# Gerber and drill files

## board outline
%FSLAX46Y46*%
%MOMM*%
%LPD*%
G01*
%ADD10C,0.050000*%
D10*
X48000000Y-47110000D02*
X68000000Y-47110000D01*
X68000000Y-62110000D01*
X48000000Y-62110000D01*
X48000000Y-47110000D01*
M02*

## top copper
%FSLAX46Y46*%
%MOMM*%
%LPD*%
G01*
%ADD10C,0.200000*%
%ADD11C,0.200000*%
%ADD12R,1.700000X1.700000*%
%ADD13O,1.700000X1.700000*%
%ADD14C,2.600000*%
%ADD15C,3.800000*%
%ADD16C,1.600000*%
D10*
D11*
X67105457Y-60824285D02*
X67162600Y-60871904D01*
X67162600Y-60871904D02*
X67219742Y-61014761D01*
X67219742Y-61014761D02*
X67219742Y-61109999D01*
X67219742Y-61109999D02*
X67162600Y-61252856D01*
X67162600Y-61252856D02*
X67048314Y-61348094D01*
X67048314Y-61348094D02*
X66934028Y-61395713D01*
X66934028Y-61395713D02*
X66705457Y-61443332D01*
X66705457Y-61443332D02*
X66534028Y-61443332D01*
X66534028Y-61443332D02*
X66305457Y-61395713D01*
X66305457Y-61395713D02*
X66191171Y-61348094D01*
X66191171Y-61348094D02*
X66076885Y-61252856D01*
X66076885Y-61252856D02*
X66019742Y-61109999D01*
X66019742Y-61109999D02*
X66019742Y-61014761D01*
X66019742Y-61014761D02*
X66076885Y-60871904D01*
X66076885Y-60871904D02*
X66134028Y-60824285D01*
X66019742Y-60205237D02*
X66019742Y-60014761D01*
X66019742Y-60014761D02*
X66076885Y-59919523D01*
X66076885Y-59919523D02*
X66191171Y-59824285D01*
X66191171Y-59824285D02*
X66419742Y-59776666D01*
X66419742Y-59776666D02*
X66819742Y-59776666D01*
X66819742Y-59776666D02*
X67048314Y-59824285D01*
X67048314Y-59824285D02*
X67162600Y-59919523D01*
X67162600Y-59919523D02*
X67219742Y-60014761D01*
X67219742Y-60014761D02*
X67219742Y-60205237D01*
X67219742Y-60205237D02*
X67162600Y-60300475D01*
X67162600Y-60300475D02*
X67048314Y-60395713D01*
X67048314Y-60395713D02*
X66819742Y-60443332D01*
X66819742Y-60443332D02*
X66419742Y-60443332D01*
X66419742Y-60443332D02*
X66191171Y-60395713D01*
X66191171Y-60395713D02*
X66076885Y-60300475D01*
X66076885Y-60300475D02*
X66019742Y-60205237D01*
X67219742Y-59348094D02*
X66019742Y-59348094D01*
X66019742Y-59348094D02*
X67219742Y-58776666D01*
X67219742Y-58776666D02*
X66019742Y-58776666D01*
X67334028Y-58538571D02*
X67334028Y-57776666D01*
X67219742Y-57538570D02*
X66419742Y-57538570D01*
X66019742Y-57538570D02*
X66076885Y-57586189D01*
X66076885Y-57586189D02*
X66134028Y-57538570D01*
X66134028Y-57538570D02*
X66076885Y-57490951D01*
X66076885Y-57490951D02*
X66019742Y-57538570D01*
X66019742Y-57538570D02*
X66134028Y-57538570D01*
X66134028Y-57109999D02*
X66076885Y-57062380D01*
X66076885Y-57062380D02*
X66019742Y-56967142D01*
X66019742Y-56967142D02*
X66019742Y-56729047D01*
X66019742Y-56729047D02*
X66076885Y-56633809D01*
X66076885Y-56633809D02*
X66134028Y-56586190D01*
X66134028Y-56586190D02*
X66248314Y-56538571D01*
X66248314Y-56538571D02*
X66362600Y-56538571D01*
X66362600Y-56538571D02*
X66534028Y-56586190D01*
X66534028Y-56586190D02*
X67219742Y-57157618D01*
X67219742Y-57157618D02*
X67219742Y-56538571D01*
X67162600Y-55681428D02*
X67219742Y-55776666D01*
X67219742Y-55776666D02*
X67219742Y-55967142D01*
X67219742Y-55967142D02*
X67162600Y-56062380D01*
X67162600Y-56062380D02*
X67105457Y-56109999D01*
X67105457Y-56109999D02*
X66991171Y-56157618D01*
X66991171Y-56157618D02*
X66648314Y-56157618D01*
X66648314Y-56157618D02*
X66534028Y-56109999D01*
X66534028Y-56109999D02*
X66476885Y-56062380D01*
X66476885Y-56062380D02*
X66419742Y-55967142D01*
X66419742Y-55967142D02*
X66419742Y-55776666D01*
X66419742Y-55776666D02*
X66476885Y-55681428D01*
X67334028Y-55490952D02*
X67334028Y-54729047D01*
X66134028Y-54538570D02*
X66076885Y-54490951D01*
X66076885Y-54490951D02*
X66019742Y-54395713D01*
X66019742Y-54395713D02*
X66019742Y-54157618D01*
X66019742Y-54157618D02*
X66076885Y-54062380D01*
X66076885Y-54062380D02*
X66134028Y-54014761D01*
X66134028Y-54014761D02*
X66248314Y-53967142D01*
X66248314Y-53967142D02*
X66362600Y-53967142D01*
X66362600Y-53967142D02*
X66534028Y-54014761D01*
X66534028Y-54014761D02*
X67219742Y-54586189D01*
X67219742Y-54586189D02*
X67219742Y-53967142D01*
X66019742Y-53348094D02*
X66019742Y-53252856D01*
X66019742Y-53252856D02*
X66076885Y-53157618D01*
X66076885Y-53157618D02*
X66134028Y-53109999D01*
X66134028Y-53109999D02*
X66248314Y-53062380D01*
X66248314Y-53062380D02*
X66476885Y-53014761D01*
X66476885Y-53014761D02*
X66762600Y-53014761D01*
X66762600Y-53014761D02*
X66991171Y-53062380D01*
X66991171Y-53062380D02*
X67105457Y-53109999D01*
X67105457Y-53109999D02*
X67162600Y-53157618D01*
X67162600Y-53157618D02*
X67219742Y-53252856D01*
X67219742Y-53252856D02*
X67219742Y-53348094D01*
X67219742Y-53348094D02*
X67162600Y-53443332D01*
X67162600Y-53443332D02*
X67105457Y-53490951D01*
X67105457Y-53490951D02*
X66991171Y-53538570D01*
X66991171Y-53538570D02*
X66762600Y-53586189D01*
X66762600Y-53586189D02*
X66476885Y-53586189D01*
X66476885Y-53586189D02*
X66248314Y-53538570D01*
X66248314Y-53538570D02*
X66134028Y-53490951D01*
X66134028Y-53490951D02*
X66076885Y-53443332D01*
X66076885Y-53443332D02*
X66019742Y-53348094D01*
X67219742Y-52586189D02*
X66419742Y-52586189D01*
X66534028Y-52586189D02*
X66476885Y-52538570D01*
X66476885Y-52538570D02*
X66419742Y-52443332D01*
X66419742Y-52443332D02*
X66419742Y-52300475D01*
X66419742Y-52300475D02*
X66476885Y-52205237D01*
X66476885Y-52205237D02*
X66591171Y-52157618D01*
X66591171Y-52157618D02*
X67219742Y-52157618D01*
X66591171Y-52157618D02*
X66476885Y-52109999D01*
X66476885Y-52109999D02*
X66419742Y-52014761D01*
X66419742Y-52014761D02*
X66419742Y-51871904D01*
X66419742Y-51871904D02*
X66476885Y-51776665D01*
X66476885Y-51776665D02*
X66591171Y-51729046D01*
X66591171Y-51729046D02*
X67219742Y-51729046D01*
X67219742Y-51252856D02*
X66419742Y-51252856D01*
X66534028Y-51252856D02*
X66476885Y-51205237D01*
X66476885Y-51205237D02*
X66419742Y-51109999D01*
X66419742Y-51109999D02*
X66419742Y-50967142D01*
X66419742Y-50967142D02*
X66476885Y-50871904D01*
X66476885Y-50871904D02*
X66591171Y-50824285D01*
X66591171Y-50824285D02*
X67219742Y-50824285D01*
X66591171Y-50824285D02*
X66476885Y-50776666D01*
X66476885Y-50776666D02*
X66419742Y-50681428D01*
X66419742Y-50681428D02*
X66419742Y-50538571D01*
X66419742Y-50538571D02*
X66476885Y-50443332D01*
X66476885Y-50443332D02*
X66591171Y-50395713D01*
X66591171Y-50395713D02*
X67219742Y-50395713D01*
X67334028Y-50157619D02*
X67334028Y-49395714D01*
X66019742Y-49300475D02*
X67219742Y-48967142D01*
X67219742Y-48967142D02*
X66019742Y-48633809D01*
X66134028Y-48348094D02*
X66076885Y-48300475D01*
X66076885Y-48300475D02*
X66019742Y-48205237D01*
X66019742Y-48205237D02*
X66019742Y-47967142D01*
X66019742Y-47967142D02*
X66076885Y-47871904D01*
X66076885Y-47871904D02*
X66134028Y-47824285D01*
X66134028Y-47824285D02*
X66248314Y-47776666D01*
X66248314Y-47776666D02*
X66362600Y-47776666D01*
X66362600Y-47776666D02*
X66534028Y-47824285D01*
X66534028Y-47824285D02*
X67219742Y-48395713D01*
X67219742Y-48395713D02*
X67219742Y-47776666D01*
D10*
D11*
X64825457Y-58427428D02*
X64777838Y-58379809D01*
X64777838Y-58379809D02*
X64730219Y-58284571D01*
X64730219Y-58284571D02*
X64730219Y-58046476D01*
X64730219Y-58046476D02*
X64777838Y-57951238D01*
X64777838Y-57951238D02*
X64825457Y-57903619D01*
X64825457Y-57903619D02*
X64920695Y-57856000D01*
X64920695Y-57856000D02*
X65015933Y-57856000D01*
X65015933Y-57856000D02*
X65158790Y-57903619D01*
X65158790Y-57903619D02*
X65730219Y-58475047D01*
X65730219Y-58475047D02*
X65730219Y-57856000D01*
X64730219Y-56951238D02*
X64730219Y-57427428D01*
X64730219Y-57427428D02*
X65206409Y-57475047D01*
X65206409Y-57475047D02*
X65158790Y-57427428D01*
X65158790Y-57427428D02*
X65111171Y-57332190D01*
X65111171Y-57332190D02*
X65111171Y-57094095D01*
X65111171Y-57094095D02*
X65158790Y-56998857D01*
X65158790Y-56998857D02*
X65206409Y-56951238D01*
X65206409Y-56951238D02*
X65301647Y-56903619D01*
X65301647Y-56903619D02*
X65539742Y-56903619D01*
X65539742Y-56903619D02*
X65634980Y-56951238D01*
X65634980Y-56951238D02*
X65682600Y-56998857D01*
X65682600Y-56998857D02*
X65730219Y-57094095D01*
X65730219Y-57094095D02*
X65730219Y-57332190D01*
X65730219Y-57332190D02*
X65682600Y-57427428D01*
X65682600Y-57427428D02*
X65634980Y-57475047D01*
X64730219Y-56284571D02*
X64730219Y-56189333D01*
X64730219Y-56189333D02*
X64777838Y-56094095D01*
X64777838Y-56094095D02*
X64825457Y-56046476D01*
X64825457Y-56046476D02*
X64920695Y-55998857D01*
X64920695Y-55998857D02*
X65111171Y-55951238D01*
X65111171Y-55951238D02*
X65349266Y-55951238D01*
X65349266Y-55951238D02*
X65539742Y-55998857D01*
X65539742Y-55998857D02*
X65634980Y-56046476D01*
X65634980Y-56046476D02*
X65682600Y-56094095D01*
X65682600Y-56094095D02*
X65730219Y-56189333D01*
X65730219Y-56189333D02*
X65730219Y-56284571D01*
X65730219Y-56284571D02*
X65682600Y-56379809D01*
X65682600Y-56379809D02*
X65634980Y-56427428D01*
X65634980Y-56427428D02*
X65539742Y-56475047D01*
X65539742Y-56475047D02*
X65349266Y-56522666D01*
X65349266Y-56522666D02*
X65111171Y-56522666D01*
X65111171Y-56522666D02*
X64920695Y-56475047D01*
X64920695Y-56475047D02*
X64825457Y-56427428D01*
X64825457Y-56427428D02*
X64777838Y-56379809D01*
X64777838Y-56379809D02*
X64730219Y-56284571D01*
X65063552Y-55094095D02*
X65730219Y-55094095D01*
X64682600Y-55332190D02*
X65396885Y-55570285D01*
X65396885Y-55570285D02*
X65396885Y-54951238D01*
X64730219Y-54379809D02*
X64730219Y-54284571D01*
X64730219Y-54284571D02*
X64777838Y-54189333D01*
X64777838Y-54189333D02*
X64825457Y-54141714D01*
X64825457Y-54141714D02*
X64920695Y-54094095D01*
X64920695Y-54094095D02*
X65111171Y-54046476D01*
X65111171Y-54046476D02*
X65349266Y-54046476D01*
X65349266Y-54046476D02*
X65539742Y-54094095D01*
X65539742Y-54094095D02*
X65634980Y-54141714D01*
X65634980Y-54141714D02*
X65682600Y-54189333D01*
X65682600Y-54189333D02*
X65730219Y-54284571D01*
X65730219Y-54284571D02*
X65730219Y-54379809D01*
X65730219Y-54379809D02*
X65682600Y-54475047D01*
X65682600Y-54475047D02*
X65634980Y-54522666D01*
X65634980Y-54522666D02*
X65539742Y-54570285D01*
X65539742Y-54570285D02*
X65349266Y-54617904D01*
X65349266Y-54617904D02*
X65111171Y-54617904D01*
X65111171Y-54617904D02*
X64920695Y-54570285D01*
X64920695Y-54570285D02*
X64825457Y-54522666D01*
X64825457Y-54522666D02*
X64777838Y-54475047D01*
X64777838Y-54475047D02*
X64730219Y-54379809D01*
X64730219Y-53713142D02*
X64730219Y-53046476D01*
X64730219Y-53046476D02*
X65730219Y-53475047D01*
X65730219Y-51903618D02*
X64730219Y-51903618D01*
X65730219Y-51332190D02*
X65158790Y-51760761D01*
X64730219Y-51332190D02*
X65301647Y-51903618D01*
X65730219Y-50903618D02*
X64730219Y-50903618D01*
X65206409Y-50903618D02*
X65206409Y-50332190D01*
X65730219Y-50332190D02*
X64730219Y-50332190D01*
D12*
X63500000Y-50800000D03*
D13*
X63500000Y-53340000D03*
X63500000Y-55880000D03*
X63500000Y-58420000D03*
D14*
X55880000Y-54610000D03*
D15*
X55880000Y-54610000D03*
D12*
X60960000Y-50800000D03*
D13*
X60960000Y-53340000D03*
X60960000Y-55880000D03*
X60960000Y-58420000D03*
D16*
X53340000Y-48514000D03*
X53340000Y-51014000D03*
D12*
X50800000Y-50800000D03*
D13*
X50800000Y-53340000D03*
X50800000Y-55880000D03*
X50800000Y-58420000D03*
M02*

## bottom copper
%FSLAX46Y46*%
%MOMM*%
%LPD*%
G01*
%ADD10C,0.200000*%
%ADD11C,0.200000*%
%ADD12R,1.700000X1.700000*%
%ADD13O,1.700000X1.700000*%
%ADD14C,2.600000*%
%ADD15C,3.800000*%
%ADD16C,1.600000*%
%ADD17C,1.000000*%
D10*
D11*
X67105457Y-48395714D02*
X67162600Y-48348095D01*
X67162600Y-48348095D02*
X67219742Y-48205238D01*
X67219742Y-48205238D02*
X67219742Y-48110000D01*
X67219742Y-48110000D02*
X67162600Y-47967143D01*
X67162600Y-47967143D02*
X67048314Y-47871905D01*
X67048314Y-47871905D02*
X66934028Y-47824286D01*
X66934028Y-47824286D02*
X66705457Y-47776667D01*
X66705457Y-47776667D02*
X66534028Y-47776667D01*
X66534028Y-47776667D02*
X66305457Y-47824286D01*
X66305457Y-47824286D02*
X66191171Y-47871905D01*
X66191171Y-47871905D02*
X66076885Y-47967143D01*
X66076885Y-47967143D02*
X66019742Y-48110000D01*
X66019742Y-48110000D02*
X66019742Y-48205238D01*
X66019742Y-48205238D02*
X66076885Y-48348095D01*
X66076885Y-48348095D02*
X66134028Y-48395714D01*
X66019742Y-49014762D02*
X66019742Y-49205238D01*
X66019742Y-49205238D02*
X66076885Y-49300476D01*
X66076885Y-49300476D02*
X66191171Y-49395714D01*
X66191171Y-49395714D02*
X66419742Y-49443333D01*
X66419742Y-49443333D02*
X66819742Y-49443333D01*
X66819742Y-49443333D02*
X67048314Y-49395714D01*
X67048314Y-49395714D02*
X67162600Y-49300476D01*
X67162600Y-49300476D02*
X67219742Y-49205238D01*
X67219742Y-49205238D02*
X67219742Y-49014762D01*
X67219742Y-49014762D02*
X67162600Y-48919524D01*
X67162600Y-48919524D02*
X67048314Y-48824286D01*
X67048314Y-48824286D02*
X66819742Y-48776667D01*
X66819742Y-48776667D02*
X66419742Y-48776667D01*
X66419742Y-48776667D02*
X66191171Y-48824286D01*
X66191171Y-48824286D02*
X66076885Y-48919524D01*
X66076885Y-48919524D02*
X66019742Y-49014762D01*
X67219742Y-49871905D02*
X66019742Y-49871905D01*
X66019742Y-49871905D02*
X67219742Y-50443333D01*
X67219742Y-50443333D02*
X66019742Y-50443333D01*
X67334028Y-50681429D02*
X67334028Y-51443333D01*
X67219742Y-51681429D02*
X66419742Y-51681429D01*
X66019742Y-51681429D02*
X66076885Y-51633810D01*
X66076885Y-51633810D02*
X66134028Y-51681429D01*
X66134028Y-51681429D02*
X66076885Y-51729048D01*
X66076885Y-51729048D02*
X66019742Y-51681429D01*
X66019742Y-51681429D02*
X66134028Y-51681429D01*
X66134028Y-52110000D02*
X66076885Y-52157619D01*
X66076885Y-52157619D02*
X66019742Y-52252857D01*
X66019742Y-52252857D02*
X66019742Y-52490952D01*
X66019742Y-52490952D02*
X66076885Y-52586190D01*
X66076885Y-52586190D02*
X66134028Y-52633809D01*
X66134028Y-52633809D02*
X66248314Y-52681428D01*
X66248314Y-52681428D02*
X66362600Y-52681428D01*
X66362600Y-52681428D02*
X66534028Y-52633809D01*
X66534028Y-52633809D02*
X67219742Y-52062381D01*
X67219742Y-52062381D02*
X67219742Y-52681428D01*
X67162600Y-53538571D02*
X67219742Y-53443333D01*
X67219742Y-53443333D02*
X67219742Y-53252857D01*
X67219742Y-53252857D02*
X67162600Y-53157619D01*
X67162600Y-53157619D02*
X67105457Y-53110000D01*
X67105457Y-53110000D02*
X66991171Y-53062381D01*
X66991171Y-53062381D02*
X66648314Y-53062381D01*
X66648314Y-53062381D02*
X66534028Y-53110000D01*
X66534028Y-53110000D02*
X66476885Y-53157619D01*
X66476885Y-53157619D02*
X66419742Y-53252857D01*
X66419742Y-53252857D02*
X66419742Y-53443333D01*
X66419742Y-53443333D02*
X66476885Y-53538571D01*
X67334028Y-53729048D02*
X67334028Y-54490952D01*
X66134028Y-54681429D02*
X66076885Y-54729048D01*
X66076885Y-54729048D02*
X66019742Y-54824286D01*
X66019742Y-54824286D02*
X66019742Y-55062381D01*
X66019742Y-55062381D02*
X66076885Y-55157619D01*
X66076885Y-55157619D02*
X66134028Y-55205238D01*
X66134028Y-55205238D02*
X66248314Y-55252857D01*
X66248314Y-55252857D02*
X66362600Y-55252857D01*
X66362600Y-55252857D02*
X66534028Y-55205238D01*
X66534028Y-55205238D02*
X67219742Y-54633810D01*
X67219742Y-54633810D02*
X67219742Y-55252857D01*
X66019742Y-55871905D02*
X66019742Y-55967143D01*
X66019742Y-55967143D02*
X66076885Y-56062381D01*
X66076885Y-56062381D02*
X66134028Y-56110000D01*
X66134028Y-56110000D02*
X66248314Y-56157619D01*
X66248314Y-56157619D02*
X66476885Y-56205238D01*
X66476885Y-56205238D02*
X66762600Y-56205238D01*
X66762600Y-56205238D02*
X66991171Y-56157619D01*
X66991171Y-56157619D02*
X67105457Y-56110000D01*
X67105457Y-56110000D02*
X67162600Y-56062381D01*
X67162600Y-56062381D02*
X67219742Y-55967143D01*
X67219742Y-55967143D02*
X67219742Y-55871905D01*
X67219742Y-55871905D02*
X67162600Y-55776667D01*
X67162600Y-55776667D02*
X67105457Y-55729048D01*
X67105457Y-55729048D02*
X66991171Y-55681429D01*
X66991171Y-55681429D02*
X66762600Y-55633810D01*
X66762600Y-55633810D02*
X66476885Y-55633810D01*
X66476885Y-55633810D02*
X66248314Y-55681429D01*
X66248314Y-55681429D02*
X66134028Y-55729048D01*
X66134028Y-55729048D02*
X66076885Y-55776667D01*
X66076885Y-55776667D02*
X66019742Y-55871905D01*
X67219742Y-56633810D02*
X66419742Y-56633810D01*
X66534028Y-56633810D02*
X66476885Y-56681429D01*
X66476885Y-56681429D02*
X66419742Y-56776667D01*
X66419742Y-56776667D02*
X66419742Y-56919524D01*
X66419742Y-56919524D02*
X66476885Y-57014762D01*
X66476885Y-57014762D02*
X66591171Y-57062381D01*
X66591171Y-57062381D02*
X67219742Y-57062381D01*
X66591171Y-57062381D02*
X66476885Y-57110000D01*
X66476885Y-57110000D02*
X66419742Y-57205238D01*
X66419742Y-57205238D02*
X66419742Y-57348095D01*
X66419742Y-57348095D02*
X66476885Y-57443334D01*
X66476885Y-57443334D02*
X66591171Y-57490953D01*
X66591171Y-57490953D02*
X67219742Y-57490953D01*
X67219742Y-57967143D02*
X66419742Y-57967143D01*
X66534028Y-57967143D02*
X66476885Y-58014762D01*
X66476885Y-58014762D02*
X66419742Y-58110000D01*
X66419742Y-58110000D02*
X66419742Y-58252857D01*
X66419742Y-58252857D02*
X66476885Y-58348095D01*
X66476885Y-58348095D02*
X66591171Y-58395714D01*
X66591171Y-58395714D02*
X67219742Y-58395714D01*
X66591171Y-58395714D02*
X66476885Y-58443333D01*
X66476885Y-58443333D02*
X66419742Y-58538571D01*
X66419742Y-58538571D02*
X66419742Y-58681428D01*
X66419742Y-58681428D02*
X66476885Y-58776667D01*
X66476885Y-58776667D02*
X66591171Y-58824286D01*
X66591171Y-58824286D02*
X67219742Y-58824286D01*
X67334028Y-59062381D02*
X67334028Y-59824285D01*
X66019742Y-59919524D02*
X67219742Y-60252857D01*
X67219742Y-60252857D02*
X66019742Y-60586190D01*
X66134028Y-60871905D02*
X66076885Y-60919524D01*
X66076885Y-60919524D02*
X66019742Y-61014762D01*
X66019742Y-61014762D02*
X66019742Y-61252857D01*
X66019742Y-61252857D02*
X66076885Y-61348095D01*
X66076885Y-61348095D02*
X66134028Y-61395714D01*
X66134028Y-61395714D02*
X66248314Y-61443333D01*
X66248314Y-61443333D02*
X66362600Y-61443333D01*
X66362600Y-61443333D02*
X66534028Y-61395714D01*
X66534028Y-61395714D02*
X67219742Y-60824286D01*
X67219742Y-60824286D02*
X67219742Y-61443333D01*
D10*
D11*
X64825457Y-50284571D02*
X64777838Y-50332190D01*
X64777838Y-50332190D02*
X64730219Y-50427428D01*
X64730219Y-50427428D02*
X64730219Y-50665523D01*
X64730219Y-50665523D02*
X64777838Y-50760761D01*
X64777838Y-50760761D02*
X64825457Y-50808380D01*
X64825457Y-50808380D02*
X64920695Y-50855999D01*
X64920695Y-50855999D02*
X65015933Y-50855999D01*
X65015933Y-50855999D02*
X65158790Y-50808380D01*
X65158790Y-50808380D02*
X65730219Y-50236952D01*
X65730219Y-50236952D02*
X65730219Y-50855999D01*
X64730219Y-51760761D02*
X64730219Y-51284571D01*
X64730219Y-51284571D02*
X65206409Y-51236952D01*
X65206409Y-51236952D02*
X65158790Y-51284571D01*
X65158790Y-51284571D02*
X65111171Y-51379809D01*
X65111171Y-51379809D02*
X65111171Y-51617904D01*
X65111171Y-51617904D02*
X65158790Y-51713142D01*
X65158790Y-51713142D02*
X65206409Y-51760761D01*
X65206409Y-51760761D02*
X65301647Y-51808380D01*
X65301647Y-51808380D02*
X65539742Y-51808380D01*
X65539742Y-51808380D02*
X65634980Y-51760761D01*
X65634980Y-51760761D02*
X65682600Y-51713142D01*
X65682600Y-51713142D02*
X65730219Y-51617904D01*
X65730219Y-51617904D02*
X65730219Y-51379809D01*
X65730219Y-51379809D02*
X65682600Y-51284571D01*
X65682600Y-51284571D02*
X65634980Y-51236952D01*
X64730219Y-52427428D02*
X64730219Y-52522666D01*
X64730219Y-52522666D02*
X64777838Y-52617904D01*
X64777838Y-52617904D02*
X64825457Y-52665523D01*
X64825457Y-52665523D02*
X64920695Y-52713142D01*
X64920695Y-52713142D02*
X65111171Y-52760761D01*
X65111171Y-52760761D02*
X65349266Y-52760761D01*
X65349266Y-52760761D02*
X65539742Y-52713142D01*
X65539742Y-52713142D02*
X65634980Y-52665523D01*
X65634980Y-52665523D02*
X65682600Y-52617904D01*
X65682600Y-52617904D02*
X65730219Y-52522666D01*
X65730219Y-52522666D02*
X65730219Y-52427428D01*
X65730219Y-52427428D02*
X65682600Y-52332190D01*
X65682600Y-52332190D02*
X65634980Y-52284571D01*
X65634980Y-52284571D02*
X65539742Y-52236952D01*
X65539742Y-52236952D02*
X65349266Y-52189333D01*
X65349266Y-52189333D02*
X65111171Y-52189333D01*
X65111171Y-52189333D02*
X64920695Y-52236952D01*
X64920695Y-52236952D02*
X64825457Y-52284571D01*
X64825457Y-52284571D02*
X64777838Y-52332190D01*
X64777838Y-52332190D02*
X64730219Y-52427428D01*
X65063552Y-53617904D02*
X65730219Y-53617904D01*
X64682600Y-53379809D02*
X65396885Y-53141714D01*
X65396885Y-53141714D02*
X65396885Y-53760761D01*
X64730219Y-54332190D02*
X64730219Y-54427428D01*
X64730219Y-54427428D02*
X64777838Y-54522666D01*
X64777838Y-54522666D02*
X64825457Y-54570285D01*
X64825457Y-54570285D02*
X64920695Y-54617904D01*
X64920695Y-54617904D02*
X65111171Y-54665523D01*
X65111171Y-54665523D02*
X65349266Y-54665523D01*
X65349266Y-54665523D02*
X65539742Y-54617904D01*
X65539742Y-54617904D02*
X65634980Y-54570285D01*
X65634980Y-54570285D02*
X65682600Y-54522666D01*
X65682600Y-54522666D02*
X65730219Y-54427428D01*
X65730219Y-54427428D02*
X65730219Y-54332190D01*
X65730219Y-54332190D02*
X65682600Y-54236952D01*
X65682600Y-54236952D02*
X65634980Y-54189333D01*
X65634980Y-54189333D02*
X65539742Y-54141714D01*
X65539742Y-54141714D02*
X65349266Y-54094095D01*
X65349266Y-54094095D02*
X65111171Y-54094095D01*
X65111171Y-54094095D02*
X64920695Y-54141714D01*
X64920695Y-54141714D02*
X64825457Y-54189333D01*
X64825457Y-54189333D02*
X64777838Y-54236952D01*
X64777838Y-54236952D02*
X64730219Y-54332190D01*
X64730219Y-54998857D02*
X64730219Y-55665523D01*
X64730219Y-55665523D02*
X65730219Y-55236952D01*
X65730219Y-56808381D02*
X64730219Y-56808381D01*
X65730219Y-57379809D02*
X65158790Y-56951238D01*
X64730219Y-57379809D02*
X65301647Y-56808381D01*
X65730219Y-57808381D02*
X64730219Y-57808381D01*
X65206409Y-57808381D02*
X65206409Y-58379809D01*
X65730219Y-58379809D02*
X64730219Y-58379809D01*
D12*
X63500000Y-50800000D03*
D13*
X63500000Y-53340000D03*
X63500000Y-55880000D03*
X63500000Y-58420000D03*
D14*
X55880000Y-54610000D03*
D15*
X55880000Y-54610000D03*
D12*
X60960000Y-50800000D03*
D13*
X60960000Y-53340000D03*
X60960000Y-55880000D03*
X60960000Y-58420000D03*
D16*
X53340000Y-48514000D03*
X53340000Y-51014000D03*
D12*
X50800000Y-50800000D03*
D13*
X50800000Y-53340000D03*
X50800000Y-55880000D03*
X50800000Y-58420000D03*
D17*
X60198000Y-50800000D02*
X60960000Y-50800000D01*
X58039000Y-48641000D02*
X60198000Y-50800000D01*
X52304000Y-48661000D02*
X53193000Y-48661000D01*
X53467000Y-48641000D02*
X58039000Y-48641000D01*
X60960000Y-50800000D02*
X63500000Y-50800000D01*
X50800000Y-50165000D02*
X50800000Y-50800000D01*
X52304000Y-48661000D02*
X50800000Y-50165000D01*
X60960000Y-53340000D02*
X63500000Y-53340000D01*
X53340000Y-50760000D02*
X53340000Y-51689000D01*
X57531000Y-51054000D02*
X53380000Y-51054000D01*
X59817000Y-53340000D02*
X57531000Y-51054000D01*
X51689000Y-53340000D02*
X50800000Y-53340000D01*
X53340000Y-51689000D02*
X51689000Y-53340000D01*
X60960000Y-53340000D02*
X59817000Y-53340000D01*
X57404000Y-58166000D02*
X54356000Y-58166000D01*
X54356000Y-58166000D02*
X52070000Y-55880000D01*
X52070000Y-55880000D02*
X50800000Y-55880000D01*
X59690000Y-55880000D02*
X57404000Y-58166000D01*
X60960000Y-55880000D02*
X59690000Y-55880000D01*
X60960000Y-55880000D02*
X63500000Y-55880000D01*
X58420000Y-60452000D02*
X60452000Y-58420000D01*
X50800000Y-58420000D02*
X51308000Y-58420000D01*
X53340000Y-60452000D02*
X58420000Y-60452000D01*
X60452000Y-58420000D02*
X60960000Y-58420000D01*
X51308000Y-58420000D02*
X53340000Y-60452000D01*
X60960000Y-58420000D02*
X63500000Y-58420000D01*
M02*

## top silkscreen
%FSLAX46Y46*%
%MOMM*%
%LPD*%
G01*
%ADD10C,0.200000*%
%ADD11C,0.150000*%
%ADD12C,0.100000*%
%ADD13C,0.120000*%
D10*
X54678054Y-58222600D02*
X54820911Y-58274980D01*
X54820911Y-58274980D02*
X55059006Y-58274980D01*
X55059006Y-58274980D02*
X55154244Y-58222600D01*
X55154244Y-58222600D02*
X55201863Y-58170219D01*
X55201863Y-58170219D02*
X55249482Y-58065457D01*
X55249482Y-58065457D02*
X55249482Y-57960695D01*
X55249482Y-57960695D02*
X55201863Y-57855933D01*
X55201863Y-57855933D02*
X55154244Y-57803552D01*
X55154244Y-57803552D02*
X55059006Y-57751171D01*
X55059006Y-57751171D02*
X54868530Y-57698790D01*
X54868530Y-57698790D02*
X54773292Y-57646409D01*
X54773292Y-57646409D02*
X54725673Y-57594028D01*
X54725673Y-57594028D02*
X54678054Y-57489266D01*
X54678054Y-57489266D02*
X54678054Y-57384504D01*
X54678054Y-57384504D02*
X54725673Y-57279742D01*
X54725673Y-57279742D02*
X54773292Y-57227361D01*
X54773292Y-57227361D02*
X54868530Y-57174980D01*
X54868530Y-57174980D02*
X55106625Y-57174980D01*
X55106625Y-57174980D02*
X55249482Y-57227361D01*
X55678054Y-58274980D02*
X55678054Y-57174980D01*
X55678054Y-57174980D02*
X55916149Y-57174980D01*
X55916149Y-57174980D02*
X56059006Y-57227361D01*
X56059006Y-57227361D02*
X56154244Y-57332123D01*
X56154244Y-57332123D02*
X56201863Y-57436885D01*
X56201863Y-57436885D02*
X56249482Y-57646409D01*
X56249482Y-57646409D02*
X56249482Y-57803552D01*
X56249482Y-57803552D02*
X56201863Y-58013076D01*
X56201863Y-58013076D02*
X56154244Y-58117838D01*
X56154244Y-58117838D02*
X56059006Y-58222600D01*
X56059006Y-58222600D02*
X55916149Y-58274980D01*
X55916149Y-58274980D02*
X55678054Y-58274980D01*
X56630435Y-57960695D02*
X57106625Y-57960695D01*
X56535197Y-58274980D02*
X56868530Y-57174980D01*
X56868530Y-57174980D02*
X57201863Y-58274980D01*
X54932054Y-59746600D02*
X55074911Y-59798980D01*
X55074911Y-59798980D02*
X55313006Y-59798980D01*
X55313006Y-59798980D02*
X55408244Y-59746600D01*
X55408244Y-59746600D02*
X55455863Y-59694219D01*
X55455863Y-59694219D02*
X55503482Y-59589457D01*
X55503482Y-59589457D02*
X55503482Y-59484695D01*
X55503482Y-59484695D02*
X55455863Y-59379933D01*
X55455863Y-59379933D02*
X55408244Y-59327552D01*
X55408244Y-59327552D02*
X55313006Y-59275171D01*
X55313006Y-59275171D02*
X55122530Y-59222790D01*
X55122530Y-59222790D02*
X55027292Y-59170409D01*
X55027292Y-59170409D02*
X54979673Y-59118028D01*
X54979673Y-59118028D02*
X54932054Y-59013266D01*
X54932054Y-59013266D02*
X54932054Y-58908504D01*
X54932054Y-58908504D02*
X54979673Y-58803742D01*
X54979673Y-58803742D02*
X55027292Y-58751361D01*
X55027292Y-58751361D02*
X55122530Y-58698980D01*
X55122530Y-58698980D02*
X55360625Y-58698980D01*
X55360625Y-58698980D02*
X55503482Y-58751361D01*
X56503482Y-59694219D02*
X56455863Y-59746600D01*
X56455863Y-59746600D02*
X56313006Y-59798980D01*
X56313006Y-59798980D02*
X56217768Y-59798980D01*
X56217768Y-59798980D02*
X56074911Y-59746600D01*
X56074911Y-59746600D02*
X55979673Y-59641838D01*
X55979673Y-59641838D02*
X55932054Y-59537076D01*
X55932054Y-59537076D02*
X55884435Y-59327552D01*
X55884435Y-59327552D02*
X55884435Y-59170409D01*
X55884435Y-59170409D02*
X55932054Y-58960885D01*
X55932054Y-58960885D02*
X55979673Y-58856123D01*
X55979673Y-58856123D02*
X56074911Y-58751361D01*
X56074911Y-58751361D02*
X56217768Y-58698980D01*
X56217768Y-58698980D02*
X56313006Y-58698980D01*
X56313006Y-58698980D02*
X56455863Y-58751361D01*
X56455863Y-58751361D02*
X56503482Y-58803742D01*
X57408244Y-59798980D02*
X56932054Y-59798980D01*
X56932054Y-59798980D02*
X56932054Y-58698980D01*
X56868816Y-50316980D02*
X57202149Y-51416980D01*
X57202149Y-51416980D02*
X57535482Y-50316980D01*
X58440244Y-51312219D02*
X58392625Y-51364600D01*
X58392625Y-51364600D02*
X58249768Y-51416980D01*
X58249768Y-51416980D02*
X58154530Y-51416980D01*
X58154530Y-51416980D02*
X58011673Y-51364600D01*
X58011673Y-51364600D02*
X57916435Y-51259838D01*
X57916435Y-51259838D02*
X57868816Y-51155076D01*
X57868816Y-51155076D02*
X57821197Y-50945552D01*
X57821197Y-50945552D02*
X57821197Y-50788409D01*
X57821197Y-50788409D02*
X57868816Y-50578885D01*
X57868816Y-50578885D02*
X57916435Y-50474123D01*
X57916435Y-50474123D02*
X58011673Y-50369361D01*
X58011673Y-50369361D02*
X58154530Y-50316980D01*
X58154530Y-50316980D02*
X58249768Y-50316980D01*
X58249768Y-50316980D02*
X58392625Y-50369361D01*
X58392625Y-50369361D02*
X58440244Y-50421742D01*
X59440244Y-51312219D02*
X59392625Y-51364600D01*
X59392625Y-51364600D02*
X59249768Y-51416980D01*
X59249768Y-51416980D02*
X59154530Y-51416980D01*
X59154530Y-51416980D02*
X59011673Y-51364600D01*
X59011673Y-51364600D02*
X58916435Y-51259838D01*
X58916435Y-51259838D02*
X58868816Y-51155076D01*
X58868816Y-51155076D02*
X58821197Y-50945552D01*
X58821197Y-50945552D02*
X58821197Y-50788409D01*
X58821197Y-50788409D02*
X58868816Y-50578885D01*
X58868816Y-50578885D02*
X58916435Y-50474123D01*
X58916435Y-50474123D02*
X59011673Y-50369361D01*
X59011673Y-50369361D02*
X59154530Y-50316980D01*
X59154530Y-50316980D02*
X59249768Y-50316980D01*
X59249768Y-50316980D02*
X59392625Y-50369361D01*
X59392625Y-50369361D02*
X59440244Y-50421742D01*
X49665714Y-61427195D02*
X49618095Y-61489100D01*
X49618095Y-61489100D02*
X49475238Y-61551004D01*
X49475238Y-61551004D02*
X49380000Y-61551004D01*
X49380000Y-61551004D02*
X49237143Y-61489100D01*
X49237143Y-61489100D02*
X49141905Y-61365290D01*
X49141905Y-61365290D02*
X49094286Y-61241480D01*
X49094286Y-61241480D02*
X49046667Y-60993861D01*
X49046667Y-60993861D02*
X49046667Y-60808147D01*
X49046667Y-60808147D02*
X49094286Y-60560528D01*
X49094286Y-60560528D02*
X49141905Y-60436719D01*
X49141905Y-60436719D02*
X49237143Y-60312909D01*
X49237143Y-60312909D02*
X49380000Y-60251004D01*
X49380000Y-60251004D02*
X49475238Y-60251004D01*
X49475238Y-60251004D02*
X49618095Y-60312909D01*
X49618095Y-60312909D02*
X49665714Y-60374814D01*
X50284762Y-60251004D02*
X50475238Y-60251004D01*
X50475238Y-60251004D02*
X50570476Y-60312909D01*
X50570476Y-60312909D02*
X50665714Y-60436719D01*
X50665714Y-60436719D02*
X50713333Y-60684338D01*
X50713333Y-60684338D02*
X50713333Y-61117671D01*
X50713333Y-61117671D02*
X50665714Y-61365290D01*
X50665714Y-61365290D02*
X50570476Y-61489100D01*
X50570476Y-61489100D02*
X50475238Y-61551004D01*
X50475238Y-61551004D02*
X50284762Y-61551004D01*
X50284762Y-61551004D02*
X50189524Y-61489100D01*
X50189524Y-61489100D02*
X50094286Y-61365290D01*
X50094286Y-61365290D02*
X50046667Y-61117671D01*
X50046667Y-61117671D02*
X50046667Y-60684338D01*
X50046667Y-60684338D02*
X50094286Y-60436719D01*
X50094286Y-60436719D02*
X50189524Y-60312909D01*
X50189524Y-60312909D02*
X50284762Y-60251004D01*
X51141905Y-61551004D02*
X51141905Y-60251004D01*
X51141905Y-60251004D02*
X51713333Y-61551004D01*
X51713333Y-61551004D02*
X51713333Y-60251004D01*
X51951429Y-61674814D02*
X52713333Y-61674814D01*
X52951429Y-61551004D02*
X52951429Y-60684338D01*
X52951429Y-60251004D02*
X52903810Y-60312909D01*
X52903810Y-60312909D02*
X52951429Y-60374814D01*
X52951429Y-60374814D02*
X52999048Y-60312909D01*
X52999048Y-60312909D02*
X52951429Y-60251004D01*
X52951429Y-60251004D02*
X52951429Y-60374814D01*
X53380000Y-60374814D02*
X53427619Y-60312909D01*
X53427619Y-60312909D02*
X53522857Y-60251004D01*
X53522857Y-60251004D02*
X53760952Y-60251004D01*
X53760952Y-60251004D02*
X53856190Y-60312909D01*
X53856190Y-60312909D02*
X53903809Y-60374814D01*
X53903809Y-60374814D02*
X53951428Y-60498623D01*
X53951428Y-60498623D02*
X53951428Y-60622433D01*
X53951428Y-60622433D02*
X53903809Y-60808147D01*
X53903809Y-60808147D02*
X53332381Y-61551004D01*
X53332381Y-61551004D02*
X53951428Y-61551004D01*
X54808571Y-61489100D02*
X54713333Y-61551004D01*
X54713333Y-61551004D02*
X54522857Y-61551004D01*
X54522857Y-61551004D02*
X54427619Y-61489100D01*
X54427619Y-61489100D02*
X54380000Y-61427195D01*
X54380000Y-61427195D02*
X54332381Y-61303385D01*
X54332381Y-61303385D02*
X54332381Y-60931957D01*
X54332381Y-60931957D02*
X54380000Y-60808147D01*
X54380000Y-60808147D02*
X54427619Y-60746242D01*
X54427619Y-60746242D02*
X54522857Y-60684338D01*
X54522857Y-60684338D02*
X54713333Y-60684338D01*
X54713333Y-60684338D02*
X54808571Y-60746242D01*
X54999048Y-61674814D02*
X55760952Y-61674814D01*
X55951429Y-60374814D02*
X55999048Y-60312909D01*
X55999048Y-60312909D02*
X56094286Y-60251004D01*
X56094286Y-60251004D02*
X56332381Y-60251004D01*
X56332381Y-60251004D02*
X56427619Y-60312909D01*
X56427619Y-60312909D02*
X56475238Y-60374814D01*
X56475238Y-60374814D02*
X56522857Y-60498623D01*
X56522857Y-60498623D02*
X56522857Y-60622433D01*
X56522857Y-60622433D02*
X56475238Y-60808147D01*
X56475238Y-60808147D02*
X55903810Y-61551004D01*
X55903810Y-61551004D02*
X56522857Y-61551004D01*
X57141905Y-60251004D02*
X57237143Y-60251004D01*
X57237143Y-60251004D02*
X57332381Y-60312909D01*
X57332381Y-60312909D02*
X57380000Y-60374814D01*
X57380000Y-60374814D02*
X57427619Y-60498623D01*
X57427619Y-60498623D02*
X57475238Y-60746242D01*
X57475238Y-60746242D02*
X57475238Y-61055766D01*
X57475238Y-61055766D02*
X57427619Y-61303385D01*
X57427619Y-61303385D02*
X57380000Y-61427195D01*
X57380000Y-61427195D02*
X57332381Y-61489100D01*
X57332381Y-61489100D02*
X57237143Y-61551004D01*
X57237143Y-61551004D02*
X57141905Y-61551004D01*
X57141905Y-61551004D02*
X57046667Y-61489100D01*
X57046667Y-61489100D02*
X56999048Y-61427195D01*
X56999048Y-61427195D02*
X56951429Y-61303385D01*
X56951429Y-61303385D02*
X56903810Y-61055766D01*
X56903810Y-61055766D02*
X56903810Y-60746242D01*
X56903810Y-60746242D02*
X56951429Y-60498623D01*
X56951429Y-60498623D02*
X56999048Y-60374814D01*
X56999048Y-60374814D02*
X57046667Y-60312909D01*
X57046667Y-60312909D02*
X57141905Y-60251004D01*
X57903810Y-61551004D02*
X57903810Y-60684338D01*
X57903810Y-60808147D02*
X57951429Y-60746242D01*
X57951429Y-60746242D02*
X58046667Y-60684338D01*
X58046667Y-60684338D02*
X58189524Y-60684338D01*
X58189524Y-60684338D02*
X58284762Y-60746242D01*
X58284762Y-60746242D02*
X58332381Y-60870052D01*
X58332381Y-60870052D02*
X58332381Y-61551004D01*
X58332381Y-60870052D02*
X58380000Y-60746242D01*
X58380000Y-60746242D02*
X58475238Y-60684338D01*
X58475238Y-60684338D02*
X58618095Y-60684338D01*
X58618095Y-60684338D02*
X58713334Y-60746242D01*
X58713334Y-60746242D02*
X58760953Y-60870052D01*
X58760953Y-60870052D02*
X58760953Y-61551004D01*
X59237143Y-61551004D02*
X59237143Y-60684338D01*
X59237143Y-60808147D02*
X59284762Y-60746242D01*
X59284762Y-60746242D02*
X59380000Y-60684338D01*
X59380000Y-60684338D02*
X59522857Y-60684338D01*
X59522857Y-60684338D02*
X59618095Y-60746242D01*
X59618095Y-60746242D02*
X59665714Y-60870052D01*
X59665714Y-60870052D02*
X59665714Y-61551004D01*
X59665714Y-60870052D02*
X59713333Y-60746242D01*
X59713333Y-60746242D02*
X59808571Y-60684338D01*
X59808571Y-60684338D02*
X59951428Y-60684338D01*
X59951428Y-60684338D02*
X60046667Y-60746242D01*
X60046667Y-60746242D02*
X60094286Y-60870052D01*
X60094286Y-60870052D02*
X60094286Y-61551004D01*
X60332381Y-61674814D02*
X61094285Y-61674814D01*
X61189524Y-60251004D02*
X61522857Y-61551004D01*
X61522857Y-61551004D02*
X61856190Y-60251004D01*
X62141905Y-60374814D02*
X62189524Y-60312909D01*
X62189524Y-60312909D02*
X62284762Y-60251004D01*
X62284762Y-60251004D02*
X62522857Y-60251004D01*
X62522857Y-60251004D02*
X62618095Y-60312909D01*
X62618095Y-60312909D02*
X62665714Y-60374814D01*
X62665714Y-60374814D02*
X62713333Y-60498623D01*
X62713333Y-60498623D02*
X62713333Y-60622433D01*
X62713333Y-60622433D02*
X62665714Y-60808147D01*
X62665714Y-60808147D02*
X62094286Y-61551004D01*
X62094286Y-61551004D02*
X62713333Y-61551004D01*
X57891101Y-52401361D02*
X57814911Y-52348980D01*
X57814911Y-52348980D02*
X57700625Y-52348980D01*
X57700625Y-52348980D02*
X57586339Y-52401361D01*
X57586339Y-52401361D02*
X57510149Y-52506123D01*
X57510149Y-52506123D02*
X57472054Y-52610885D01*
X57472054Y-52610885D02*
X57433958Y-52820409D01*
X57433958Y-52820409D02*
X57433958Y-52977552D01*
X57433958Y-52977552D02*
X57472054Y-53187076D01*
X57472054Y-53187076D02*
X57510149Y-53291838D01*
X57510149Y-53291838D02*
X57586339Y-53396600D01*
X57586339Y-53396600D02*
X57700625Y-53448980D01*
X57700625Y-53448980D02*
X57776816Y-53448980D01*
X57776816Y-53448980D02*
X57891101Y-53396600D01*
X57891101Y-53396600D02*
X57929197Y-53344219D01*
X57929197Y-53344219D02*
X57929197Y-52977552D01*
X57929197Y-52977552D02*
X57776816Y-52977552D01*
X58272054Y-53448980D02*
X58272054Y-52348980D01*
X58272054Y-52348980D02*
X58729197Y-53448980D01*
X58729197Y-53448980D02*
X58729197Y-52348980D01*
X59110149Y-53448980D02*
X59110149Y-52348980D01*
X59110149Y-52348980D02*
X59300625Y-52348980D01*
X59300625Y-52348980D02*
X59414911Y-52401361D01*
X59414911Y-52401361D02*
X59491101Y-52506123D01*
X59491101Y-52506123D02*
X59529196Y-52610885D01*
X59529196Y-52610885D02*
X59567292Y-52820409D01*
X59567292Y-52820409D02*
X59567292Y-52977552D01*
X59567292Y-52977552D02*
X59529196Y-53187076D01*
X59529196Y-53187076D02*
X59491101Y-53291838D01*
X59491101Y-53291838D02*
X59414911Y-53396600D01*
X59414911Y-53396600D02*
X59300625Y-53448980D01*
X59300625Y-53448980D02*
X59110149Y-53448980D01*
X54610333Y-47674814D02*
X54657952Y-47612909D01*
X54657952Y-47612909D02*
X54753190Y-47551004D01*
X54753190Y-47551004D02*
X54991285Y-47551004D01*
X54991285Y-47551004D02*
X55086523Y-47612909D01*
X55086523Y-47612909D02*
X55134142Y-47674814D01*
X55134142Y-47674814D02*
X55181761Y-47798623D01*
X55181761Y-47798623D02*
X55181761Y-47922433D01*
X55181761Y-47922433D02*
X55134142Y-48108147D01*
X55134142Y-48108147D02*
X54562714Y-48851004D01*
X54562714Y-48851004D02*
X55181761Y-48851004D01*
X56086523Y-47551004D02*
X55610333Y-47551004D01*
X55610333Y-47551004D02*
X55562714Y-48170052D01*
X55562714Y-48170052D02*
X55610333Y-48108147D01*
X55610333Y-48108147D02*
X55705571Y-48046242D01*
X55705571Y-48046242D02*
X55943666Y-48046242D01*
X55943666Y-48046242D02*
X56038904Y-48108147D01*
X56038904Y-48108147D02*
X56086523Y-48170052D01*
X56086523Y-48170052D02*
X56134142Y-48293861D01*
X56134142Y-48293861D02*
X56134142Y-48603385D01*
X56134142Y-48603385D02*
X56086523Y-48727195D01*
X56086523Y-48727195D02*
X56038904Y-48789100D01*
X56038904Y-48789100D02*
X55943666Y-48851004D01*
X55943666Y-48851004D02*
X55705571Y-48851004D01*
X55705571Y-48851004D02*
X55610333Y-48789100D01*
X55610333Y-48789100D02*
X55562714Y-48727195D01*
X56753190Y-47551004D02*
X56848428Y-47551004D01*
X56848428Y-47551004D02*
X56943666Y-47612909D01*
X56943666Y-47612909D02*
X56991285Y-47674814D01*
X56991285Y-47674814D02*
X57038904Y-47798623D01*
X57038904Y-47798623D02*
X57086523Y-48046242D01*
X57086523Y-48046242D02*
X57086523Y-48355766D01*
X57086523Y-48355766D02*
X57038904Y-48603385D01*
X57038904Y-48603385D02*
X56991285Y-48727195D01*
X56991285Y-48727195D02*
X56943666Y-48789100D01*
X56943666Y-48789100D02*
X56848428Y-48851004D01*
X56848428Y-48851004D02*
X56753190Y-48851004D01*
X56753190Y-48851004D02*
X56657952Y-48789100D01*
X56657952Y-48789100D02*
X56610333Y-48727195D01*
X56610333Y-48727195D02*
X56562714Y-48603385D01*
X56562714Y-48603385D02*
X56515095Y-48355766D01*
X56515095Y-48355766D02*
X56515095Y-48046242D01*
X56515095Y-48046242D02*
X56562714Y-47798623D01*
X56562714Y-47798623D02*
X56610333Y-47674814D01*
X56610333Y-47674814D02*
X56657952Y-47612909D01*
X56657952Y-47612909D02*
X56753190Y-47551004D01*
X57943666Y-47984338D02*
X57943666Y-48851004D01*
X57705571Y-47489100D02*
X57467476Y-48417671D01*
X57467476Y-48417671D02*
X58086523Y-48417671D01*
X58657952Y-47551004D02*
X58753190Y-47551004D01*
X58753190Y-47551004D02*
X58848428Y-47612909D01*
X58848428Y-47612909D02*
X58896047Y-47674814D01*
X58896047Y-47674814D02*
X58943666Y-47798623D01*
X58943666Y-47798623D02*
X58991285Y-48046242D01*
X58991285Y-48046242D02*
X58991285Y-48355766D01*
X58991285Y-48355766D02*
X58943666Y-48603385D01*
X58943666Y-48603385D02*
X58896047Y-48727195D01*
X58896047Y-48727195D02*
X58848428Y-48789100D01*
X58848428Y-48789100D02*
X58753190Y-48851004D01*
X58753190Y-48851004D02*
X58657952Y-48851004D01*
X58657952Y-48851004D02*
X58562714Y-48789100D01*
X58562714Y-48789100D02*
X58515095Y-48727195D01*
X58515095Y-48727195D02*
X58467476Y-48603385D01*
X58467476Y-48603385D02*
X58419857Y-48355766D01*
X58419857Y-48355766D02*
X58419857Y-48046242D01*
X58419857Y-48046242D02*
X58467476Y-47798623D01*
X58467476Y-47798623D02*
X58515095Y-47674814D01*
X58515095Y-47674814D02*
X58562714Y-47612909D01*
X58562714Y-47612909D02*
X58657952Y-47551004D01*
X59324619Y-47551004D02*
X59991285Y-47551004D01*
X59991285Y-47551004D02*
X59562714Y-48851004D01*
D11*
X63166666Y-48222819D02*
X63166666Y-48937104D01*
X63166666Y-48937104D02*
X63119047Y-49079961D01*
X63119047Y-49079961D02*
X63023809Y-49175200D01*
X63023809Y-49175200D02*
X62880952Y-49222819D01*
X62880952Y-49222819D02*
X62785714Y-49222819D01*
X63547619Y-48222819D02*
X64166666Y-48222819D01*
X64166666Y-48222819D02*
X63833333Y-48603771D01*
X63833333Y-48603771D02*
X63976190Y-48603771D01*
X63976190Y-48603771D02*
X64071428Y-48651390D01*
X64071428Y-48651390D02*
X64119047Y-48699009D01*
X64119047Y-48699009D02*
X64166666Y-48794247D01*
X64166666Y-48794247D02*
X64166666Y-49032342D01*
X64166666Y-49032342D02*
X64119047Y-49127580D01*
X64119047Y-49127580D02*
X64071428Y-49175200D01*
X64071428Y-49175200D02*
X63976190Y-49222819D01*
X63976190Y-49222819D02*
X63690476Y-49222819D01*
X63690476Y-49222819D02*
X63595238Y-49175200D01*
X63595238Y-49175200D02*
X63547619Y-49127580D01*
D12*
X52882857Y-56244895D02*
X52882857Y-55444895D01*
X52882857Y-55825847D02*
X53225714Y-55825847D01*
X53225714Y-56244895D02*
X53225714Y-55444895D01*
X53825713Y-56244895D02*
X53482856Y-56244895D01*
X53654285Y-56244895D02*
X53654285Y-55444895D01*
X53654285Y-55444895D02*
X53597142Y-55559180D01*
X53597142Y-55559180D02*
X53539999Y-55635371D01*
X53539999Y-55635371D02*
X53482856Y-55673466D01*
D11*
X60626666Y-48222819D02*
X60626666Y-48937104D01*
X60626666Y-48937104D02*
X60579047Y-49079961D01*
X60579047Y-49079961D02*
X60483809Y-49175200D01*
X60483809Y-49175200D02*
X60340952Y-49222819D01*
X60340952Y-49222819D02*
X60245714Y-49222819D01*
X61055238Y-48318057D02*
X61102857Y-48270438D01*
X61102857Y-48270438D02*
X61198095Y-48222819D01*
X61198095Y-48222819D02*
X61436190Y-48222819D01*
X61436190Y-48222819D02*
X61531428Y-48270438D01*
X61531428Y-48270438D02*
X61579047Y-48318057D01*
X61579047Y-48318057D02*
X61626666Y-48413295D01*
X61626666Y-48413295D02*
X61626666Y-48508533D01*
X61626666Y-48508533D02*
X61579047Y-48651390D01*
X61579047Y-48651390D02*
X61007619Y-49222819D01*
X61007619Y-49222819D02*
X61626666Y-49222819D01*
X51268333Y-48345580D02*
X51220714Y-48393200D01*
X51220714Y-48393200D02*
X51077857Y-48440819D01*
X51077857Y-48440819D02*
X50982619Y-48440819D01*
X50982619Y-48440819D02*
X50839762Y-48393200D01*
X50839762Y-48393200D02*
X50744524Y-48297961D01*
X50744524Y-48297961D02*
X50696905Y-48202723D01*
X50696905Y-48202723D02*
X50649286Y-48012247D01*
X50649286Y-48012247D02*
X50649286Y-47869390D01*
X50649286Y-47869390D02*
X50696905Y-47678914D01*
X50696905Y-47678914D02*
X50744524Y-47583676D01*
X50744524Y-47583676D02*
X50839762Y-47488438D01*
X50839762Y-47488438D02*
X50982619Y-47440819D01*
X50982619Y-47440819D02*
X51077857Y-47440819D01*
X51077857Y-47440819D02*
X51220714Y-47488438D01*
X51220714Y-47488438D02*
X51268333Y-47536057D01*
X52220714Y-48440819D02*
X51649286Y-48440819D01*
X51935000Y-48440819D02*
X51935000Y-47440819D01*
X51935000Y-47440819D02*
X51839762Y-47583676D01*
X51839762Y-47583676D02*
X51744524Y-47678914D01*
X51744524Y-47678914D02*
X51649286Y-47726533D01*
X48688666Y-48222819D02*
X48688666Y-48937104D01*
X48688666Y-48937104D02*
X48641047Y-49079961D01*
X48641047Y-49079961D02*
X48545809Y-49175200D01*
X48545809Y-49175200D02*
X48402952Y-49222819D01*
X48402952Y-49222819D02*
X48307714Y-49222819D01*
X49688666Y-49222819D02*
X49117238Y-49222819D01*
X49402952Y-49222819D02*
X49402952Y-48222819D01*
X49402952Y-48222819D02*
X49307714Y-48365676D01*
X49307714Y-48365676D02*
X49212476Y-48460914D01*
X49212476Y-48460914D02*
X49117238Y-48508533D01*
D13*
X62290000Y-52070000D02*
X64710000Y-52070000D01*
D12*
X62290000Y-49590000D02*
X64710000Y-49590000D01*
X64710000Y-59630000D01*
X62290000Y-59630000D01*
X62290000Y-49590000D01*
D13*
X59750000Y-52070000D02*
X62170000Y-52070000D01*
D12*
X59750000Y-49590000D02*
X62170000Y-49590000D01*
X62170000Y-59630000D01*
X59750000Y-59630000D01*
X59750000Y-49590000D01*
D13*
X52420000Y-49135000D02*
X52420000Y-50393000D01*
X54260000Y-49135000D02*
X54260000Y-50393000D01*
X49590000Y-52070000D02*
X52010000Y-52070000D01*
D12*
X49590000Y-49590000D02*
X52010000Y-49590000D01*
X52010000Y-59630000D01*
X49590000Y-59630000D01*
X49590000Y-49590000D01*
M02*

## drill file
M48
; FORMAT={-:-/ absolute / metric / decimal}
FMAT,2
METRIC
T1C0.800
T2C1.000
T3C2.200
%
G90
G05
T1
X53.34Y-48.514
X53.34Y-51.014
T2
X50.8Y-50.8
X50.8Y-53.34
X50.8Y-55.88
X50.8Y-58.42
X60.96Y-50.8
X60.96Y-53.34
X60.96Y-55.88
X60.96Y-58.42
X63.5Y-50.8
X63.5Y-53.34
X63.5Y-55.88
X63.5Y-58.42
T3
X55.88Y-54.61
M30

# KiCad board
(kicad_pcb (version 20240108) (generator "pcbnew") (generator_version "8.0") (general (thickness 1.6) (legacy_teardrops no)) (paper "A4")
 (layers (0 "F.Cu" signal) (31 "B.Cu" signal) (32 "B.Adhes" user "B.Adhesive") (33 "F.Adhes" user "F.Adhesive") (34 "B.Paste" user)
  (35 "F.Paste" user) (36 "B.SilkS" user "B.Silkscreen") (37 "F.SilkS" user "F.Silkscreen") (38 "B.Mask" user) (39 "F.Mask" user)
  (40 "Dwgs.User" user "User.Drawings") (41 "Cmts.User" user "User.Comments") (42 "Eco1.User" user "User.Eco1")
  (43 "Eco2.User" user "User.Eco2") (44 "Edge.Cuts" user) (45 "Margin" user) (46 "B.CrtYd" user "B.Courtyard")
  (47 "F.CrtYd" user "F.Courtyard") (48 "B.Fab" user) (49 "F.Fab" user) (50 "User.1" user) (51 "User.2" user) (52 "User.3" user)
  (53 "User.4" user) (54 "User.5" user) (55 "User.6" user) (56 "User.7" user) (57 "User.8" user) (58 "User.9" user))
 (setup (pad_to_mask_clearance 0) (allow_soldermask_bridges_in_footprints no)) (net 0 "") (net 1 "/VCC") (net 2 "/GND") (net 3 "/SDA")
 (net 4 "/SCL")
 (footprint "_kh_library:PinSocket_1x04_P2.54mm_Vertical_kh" (layer "F.Cu") (at 63.5 50.8)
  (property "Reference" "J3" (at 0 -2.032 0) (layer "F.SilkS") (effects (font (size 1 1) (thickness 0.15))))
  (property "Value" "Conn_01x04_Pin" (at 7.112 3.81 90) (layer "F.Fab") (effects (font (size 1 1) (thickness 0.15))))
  (fp_line (start -1.21 1.27) (end 1.21 1.27) (stroke (width 0.12) (type solid)) (layer "F.SilkS"))
  (fp_rect (start -1.21 -1.21) (end 1.21 8.83) (stroke (width 0.1) (type default)) (fill none) (layer "F.SilkS"))
  (pad "1" thru_hole rect (at 0 0) (size 1.7 1.7) (drill 1) (layers "*.Cu" "*.Mask") (remove_unused_layers no) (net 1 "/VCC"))
  (pad "2" thru_hole oval (at 0 2.54) (size 1.7 1.7) (drill 1) (layers "*.Cu" "*.Mask") (remove_unused_layers no) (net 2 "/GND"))
  (pad "3" thru_hole oval (at 0 5.08) (size 1.7 1.7) (drill 1) (layers "*.Cu" "*.Mask") (remove_unused_layers no) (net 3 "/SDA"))
  (pad "4" thru_hole oval (at 0 7.62) (size 1.7 1.7) (drill 1) (layers "*.Cu" "*.Mask") (remove_unused_layers no) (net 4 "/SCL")))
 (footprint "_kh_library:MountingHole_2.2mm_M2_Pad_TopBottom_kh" (layer "F.Cu") (at 55.88 54.61)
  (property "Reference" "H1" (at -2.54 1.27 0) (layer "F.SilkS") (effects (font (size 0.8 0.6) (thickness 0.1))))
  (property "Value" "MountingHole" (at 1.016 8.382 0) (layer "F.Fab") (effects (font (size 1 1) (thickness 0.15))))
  (pad "1" thru_hole circle (at 0 0) (size 2.6 2.6) (drill 2.2) (layers "*.Cu" "*.Mask") (remove_unused_layers no))
  (pad "1" connect circle (at 0 0) (size 3.8 3.8) (layers "F.Cu" "F.Mask"))
  (pad "1" connect circle (at 0 0) (size 3.8 3.8) (layers "B.Cu" "B.Mask")))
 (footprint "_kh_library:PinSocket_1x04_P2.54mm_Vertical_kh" (layer "F.Cu") (at 60.96 50.8)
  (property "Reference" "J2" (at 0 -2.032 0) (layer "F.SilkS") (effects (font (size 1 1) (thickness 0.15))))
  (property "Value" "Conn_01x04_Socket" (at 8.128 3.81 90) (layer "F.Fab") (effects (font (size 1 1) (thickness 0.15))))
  (fp_line (start -1.21 1.27) (end 1.21 1.27) (stroke (width 0.12) (type solid)) (layer "F.SilkS"))
  (fp_rect (start -1.21 -1.21) (end 1.21 8.83) (stroke (width 0.1) (type default)) (fill none) (layer "F.SilkS"))
  (pad "1" thru_hole rect (at 0 0) (size 1.7 1.7) (drill 1) (layers "*.Cu" "*.Mask") (remove_unused_layers no) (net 1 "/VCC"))
  (pad "2" thru_hole oval (at 0 2.54) (size 1.7 1.7) (drill 1) (layers "*.Cu" "*.Mask") (remove_unused_layers no) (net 2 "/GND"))
  (pad "3" thru_hole oval (at 0 5.08) (size 1.7 1.7) (drill 1) (layers "*.Cu" "*.Mask") (remove_unused_layers no) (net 3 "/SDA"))
  (pad "4" thru_hole oval (at 0 7.62) (size 1.7 1.7) (drill 1) (layers "*.Cu" "*.Mask") (remove_unused_layers no) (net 4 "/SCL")))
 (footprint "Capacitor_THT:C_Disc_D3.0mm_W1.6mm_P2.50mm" (layer "F.Cu") (at 53.34 48.514 -90)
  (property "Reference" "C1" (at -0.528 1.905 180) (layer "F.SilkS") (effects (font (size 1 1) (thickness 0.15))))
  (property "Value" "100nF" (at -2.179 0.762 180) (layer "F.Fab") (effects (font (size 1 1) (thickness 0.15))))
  (fp_line (start 0.621 0.92) (end 1.879 0.92) (stroke (width 0.12) (type solid)) (layer "F.SilkS"))
  (fp_line (start 0.621 -0.92) (end 1.879 -0.92) (stroke (width 0.12) (type solid)) (layer "F.SilkS"))
  (pad "1" thru_hole circle (at 0 0 270) (size 1.6 1.6) (drill 0.8) (layers "*.Cu" "*.Mask") (remove_unused_layers no) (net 1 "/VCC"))
  (pad "2" thru_hole circle (at 2.5 0 270) (size 1.6 1.6) (drill 0.8) (layers "*.Cu" "*.Mask") (remove_unused_layers no) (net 2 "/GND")))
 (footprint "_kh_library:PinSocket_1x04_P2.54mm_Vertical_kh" (layer "F.Cu") (at 50.8 50.8)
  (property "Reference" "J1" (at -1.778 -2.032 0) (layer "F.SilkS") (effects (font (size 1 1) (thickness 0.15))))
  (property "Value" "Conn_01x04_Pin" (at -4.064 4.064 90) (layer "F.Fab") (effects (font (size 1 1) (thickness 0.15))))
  (fp_line (start -1.21 1.27) (end 1.21 1.27) (stroke (width 0.12) (type solid)) (layer "F.SilkS"))
  (fp_rect (start -1.21 -1.21) (end 1.21 8.83) (stroke (width 0.1) (type default)) (fill none) (layer "F.SilkS"))
  (pad "1" thru_hole rect (at 0 0) (size 1.7 1.7) (drill 1) (layers "*.Cu" "*.Mask") (remove_unused_layers no) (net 1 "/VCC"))
  (pad "2" thru_hole oval (at 0 2.54) (size 1.7 1.7) (drill 1) (layers "*.Cu" "*.Mask") (remove_unused_layers no) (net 2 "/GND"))
  (pad "3" thru_hole oval (at 0 5.08) (size 1.7 1.7) (drill 1) (layers "*.Cu" "*.Mask") (remove_unused_layers no) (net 3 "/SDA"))
  (pad "4" thru_hole oval (at 0 7.62) (size 1.7 1.7) (drill 1) (layers "*.Cu" "*.Mask") (remove_unused_layers no) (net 4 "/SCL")))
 (gr_rect (start 48 47.11) (end 68 62.11) (stroke (width 0.05) (type default)) (fill none) (layer "Edge.Cuts"))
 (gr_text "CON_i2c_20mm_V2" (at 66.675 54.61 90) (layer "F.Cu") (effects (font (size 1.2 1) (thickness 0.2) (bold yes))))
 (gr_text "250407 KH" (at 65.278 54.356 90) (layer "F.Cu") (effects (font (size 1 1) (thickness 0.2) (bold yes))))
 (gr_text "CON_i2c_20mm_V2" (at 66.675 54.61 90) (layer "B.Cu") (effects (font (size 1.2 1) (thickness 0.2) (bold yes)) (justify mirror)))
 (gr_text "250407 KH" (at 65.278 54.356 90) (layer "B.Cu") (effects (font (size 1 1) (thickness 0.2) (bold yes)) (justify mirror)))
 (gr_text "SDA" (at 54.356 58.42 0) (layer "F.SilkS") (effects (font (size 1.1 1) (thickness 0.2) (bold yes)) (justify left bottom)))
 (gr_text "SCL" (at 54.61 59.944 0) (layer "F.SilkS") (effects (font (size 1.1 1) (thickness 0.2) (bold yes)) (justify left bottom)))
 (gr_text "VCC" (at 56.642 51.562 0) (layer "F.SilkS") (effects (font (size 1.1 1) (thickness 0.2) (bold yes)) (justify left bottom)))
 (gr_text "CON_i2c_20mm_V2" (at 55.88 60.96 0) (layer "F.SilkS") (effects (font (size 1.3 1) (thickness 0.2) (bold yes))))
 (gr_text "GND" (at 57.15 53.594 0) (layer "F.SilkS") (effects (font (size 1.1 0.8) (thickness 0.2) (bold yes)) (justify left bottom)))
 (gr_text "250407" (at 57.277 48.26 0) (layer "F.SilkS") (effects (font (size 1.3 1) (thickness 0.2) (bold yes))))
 (segment (start 60.198 50.8) (end 60.96 50.8) (width 1) (layer "B.Cu") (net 1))
 (segment (start 58.039 48.641) (end 60.198 50.8) (width 1) (layer "B.Cu") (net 1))
 (segment (start 52.304 48.661) (end 53.193 48.661) (width 1) (layer "B.Cu") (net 1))
 (segment (start 53.467 48.641) (end 58.039 48.641) (width 1) (layer "B.Cu") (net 1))
 (segment (start 60.96 50.8) (end 63.5 50.8) (width 1) (layer "B.Cu") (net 1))
 (segment (start 50.8 50.165) (end 50.8 50.8) (width 1) (layer "B.Cu") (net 1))
 (segment (start 52.304 48.661) (end 50.8 50.165) (width 1) (layer "B.Cu") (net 1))
 (segment (start 60.96 53.34) (end 63.5 53.34) (width 1) (layer "B.Cu") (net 2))
 (segment (start 53.34 50.76) (end 53.34 51.689) (width 1) (layer "B.Cu") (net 2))
 (segment (start 57.531 51.054) (end 53.38 51.054) (width 1) (layer "B.Cu") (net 2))
 (segment (start 59.817 53.34) (end 57.531 51.054) (width 1) (layer "B.Cu") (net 2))
 (segment (start 51.689 53.34) (end 50.8 53.34) (width 1) (layer "B.Cu") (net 2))
 (segment (start 53.34 51.689) (end 51.689 53.34) (width 1) (layer "B.Cu") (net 2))
 (segment (start 60.96 53.34) (end 59.817 53.34) (width 1) (layer "B.Cu") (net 2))
 (segment (start 57.404 58.166) (end 54.356 58.166) (width 1) (layer "B.Cu") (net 3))
 (segment (start 54.356 58.166) (end 52.07 55.88) (width 1) (layer "B.Cu") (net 3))
 (segment (start 52.07 55.88) (end 50.8 55.88) (width 1) (layer "B.Cu") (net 3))
 (segment (start 59.69 55.88) (end 57.404 58.166) (width 1) (layer "B.Cu") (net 3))
 (segment (start 60.96 55.88) (end 59.69 55.88) (width 1) (layer "B.Cu") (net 3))
 (segment (start 60.96 55.88) (end 63.5 55.88) (width 1) (layer "B.Cu") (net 3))
 (segment (start 58.42 60.452) (end 60.452 58.42) (width 1) (layer "B.Cu") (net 4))
 (segment (start 50.8 58.42) (end 51.308 58.42) (width 1) (layer "B.Cu") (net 4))
 (segment (start 53.34 60.452) (end 58.42 60.452) (width 1) (layer "B.Cu") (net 4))
 (segment (start 60.452 58.42) (end 60.96 58.42) (width 1) (layer "B.Cu") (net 4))
 (segment (start 51.308 58.42) (end 53.34 60.452) (width 1) (layer "B.Cu") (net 4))
 (segment (start 60.96 58.42) (end 63.5 58.42) (width 1) (layer "B.Cu") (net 4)))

